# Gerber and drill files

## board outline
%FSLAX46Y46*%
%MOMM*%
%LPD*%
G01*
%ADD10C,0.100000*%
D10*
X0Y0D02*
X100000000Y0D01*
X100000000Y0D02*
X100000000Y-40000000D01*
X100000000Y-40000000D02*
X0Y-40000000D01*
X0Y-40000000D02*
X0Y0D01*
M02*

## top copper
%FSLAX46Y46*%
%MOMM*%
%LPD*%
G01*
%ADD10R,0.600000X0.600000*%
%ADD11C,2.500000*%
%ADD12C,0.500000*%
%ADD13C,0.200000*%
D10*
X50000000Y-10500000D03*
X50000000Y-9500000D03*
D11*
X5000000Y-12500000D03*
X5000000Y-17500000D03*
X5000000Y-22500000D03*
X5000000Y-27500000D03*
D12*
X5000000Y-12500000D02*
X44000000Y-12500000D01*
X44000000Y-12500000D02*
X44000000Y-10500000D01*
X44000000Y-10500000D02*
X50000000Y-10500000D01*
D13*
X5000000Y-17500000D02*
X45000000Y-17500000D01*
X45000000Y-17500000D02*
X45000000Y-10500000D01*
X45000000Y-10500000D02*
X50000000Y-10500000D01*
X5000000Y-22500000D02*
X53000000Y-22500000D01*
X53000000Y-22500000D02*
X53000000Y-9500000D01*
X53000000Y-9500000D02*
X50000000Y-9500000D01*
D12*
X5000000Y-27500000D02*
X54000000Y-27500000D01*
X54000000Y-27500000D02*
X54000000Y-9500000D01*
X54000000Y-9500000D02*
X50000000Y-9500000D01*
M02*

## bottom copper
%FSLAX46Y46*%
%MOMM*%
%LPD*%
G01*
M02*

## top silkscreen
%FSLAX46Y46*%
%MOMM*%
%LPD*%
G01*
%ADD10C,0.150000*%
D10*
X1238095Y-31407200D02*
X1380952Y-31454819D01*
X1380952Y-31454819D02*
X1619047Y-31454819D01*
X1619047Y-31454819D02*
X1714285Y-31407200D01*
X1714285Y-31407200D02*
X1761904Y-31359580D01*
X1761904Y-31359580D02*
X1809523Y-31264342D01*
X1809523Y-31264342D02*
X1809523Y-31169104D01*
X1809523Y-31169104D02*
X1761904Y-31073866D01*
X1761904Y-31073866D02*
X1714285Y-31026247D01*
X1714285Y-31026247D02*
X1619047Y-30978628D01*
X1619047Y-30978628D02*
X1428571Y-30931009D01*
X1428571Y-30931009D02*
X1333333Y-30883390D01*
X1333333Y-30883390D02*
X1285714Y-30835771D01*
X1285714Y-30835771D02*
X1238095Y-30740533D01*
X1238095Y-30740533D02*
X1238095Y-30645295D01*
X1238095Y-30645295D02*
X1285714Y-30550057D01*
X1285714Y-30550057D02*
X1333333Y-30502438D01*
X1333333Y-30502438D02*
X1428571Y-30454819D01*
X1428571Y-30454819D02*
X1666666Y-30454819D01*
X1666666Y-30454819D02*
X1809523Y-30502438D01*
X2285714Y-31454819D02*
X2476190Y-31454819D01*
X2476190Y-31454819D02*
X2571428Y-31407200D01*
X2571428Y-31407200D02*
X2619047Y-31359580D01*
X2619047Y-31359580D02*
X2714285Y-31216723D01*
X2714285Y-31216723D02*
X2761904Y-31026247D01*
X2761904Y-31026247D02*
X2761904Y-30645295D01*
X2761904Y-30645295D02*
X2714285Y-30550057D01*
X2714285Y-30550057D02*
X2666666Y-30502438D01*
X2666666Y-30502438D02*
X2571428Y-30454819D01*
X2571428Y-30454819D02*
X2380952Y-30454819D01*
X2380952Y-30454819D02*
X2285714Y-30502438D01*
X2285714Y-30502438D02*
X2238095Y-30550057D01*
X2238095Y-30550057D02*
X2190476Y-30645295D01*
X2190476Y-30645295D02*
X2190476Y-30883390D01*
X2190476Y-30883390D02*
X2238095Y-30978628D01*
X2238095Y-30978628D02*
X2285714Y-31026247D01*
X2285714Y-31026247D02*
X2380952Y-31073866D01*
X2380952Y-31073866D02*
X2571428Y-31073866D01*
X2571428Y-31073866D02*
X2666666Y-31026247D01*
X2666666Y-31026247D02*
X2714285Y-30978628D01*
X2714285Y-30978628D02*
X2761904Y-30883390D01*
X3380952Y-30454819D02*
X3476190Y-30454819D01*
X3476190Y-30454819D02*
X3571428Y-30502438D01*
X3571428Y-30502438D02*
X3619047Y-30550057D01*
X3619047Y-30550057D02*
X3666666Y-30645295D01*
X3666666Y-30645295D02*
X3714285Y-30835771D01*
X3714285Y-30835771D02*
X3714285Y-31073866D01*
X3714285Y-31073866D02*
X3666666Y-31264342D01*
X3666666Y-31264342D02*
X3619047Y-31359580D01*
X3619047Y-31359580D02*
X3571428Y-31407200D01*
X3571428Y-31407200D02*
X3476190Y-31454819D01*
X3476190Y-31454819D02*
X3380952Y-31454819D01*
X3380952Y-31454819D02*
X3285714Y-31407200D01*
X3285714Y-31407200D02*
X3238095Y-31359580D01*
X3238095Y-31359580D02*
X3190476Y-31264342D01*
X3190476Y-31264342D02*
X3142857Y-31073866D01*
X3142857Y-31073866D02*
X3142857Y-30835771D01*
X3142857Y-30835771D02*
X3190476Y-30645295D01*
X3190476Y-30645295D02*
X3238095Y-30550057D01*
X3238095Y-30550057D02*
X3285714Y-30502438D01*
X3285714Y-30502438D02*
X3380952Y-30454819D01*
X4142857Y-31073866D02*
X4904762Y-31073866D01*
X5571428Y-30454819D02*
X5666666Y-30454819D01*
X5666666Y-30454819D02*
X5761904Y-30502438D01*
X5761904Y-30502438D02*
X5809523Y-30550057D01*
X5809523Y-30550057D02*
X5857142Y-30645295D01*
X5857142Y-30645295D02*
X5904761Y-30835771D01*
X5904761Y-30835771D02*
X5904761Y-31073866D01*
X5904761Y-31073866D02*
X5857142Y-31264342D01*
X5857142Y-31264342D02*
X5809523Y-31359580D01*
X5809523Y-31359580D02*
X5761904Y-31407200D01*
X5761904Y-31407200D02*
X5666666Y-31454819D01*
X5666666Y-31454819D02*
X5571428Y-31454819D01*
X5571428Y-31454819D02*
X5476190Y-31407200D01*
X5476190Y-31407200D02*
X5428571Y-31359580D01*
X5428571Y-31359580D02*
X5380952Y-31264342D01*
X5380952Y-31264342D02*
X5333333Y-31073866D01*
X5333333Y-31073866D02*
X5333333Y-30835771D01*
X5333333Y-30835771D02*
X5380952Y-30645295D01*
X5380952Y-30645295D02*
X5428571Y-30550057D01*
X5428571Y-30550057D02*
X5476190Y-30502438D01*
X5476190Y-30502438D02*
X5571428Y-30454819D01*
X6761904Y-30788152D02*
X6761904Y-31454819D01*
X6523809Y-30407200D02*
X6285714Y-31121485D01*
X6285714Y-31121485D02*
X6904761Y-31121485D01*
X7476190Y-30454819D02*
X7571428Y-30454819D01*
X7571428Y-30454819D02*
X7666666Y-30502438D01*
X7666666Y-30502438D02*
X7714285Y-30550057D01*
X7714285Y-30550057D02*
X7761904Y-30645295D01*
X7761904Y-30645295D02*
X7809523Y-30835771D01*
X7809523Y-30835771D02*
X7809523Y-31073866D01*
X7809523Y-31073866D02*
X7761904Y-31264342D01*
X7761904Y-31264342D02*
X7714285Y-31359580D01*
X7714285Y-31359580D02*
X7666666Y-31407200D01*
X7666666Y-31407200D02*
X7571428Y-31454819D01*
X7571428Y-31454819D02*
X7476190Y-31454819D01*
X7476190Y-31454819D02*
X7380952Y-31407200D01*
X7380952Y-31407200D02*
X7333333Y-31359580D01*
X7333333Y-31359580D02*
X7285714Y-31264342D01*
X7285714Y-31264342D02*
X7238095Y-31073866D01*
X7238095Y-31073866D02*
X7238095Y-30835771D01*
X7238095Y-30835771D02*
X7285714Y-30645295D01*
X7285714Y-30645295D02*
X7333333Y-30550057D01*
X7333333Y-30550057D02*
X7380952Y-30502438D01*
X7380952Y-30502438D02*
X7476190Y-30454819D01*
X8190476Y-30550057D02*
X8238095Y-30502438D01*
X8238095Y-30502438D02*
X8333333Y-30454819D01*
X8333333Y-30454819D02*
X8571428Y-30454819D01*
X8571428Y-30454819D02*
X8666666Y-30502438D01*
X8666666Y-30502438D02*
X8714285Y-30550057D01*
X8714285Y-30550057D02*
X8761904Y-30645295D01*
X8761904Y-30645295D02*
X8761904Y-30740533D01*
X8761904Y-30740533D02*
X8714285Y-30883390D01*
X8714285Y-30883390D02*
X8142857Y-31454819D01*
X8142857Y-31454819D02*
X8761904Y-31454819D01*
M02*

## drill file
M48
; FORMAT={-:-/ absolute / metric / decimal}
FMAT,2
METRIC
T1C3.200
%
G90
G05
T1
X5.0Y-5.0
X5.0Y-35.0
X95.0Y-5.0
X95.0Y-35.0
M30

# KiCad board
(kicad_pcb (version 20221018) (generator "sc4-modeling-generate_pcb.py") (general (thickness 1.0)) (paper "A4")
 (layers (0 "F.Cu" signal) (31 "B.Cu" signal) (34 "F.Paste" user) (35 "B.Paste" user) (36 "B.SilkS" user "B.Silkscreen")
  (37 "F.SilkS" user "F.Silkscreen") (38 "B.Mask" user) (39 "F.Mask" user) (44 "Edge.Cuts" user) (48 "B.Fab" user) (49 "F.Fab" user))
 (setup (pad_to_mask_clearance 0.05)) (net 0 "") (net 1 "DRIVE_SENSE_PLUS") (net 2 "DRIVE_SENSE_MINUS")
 (gr_line (start 0.0 0.0) (end 100.0 0.0) (layer "Edge.Cuts") (width 0.1))
 (gr_line (start 100.0 0.0) (end 100.0 40.0) (layer "Edge.Cuts") (width 0.1))
 (gr_line (start 100.0 40.0) (end 0.0 40.0) (layer "Edge.Cuts") (width 0.1))
 (gr_line (start 0.0 40.0) (end 0.0 0.0) (layer "Edge.Cuts") (width 0.1))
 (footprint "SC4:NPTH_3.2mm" (layer "F.Cu") (at 5.0 5.0)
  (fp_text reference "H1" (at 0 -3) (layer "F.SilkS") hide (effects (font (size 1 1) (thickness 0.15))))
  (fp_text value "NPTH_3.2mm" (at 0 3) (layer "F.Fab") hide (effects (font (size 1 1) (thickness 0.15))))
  (pad "1" np_thru_hole circle (at 0 0) (size 3.2 3.2) (drill 3.2) (layers "*.Cu" "*.Mask")))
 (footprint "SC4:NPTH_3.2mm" (layer "F.Cu") (at 95.0 5.0)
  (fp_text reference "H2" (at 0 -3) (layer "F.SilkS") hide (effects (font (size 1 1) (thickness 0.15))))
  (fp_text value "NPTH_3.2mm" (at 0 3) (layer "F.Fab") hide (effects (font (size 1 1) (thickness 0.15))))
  (pad "1" np_thru_hole circle (at 0 0) (size 3.2 3.2) (drill 3.2) (layers "*.Cu" "*.Mask")))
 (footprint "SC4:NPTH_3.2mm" (layer "F.Cu") (at 5.0 35.0)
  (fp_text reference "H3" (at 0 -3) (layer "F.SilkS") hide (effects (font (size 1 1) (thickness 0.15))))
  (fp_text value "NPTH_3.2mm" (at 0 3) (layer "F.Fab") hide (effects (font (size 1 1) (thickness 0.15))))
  (pad "1" np_thru_hole circle (at 0 0) (size 3.2 3.2) (drill 3.2) (layers "*.Cu" "*.Mask")))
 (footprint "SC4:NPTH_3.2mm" (layer "F.Cu") (at 95.0 35.0)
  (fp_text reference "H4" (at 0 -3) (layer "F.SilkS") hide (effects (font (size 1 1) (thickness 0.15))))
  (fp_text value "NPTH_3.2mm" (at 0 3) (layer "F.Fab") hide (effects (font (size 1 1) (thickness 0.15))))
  (pad "1" np_thru_hole circle (at 0 0) (size 3.2 3.2) (drill 3.2) (layers "*.Cu" "*.Mask")))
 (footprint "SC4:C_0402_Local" (layer "F.Cu") (at 50.0 10.0 90)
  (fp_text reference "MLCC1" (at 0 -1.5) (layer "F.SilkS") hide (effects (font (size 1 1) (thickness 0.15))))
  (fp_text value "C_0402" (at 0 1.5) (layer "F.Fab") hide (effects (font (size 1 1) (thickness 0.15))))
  (pad "1" smd rect (at -0.5 0) (size 0.6 0.6) (layers "F.Cu" "F.Paste" "F.Mask") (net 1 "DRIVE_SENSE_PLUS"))
  (pad "2" smd rect (at 0.5 0) (size 0.6 0.6) (layers "F.Cu" "F.Paste" "F.Mask") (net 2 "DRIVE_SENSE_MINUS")))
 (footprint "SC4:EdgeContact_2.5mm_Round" (layer "F.Cu") (at 5.0 12.5)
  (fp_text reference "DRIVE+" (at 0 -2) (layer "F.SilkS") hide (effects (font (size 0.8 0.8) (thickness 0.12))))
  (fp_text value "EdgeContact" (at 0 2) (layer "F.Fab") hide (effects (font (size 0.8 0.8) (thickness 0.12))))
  (pad "1" smd circle (at 0 0) (size 2.5 2.5) (layers "F.Cu" "F.Mask") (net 1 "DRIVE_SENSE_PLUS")))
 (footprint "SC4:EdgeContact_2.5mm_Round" (layer "F.Cu") (at 5.0 17.5)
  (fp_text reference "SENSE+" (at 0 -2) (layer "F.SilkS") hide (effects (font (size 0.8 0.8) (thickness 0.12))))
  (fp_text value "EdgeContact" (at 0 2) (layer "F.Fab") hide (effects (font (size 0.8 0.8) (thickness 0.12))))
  (pad "1" smd circle (at 0 0) (size 2.5 2.5) (layers "F.Cu" "F.Mask") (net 1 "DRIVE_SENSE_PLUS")))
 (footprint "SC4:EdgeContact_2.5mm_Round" (layer "F.Cu") (at 5.0 22.5)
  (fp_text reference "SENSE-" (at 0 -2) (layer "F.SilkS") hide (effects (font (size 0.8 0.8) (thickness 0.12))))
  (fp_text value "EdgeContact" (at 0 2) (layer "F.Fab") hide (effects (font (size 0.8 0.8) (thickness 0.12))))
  (pad "1" smd circle (at 0 0) (size 2.5 2.5) (layers "F.Cu" "F.Mask") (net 2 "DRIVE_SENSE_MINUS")))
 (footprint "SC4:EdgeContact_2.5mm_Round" (layer "F.Cu") (at 5.0 27.5)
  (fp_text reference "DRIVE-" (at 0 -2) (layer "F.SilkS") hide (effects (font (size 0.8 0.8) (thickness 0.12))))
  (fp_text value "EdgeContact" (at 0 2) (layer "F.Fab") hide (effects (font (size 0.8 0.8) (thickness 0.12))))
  (pad "1" smd circle (at 0 0) (size 2.5 2.5) (layers "F.Cu" "F.Mask") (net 2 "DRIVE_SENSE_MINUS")))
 (segment (start 5.0 12.5) (end 44.0 12.5) (width 0.5) (layer "F.Cu") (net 1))
 (segment (start 44.0 12.5) (end 44.0 10.5) (width 0.5) (layer "F.Cu") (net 1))
 (segment (start 44.0 10.5) (end 50.0 10.5) (width 0.5) (layer "F.Cu") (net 1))
 (segment (start 5.0 17.5) (end 45.0 17.5) (width 0.2) (layer "F.Cu") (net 1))
 (segment (start 45.0 17.5) (end 45.0 10.5) (width 0.2) (layer "F.Cu") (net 1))
 (segment (start 45.0 10.5) (end 50.0 10.5) (width 0.2) (layer "F.Cu") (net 1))
 (segment (start 5.0 22.5) (end 53.0 22.5) (width 0.2) (layer "F.Cu") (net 2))
 (segment (start 53.0 22.5) (end 53.0 9.5) (width 0.2) (layer "F.Cu") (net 2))
 (segment (start 53.0 9.5) (end 50.0 9.5) (width 0.2) (layer "F.Cu") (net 2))
 (segment (start 5.0 27.5) (end 54.0 27.5) (width 0.5) (layer "F.Cu") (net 2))
 (segment (start 54.0 27.5) (end 54.0 9.5) (width 0.5) (layer "F.Cu") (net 2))
 (segment (start 54.0 9.5) (end 50.0 9.5) (width 0.5) (layer "F.Cu") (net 2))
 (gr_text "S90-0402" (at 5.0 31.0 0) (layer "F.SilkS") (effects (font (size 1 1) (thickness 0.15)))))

